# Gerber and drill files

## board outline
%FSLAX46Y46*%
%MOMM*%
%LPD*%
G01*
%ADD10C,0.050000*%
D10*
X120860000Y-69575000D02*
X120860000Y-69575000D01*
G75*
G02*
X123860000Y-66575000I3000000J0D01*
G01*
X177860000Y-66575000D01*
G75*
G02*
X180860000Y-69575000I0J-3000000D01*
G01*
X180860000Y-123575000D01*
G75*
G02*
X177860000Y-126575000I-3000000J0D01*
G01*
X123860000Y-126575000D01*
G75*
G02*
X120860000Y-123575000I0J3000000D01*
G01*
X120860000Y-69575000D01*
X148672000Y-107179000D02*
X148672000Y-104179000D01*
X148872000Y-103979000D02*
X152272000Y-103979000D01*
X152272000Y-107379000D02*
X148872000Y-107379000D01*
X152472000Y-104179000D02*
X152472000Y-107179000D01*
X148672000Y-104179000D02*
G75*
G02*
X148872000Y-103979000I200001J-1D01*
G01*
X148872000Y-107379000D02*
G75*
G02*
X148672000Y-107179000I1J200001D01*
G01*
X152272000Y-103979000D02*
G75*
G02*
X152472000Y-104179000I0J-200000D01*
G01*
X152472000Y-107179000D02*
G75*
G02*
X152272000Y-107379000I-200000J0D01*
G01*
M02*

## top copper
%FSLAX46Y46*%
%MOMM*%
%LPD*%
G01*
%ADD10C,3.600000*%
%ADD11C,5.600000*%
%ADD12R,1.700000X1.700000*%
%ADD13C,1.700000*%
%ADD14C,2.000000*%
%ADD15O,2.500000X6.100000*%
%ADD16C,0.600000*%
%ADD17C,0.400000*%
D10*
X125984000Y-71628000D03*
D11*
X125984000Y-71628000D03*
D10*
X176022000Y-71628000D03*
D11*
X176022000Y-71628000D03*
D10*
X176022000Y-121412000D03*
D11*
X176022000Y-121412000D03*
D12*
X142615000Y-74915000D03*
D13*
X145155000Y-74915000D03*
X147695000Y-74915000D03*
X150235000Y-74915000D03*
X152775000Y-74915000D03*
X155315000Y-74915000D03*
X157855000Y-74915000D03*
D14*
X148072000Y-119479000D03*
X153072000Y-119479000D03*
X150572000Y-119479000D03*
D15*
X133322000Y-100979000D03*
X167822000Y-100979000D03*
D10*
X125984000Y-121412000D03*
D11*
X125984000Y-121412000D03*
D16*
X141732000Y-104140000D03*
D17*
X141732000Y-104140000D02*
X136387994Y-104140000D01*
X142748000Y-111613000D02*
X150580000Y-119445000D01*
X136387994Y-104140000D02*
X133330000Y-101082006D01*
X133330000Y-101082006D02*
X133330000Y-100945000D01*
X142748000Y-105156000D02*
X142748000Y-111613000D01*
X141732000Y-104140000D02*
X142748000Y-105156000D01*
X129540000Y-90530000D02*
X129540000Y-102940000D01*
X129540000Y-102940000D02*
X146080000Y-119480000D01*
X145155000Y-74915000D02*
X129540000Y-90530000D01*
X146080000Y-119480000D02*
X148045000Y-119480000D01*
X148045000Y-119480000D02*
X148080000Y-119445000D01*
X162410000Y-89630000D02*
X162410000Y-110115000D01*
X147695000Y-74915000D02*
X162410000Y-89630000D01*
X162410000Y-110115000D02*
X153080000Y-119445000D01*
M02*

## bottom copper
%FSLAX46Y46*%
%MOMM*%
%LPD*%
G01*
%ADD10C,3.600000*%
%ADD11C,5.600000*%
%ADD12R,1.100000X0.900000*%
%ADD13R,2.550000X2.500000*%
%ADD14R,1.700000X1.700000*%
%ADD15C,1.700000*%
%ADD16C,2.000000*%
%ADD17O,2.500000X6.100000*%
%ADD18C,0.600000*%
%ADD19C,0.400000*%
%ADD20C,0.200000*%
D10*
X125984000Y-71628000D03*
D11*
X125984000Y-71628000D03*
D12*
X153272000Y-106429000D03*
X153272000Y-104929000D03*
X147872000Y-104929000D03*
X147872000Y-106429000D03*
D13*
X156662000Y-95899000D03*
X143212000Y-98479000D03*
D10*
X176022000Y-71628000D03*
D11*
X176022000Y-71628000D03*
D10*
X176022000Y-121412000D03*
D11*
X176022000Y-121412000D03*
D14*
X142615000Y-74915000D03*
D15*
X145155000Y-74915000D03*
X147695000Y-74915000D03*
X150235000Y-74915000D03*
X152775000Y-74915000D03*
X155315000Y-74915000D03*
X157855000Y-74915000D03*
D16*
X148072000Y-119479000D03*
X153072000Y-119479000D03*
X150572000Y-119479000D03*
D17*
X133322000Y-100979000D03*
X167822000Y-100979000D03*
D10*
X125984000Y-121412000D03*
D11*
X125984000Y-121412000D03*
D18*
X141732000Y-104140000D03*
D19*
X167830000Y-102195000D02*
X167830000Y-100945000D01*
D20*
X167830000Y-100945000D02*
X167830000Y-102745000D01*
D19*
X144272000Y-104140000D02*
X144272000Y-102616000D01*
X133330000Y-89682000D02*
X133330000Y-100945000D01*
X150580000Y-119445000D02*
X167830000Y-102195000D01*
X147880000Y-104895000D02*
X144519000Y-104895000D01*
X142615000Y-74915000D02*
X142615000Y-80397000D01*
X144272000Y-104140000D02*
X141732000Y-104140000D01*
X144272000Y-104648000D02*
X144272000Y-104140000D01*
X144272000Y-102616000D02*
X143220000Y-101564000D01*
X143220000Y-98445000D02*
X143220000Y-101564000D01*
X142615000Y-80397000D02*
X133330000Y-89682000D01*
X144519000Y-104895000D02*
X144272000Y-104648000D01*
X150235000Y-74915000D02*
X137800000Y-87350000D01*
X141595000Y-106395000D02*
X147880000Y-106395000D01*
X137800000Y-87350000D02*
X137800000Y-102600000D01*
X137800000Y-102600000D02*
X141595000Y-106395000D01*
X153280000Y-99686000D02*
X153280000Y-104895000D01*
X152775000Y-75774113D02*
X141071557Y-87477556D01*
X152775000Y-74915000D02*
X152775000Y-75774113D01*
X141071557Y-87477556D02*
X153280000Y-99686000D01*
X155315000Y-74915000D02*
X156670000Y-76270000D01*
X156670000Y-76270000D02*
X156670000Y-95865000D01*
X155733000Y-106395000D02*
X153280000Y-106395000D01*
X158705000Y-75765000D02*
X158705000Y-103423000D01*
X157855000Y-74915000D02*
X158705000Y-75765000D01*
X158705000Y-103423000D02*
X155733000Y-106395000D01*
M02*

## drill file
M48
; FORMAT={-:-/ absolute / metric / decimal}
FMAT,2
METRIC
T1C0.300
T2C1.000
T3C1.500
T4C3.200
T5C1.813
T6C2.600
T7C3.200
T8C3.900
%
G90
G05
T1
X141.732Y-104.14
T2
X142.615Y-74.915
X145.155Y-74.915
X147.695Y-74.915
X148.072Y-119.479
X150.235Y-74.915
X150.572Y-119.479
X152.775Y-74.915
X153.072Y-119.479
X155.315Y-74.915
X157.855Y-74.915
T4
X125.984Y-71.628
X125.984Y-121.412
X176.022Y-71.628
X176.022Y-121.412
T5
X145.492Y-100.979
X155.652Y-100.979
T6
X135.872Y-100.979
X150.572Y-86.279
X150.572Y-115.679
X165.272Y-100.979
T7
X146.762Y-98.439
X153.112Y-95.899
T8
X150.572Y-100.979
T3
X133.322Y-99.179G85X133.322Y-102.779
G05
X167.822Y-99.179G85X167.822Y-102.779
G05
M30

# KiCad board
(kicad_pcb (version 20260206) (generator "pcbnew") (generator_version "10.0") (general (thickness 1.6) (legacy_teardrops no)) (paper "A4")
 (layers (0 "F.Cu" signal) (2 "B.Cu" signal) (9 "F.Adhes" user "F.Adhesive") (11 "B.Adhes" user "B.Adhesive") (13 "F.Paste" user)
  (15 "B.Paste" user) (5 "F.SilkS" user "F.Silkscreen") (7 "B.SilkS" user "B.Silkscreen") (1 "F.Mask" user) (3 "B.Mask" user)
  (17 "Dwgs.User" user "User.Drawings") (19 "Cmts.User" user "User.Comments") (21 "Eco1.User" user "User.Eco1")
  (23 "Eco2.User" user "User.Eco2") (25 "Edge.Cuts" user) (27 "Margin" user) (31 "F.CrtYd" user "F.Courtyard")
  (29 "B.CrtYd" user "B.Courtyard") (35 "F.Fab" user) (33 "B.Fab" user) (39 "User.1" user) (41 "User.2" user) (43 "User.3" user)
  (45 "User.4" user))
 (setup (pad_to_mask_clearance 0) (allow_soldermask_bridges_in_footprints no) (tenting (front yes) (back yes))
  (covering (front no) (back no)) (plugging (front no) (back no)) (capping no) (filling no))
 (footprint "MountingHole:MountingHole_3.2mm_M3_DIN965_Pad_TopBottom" (layer "F.Cu") (at 125.984 71.628)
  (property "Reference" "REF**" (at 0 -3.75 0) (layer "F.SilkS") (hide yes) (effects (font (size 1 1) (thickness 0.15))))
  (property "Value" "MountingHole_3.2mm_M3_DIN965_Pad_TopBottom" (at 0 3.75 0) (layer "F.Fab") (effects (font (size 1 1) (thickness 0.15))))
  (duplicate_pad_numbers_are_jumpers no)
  (pad "1" thru_hole circle (at 0 0) (size 3.6 3.6) (drill 3.2) (layers "*.Cu" "*.Mask") (remove_unused_layers no) (zone_connect 2))
  (pad "1" connect circle (at 0 0) (size 5.6 5.6) (layers "F.Cu" "F.Mask") (zone_connect 2))
  (pad "1" connect circle (at 0 0) (size 5.6 5.6) (layers "B.Cu" "B.Mask") (zone_connect 2)))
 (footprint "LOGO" (layer "F.Cu") (at 170.18 84.074 -8)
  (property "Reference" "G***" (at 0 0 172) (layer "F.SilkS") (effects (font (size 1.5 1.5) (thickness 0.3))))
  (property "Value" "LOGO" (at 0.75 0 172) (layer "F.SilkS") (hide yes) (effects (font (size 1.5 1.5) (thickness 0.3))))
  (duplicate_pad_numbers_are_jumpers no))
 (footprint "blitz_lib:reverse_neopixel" (layer "F.Cu") (at 150.572 100.979)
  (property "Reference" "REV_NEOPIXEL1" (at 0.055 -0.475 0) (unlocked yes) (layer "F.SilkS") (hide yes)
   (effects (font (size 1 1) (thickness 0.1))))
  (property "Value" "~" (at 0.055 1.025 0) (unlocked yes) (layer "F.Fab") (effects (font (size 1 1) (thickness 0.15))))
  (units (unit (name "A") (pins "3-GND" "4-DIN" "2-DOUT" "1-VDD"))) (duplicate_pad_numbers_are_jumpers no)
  (fp_line (start -1.9 6.2) (end -1.9 3.2) (stroke (width 0.05) (type solid)) (layer "Edge.Cuts"))
  (fp_line (start -1.7 3) (end 1.7 3) (stroke (width 0.05) (type solid)) (layer "Edge.Cuts"))
  (fp_line (start 1.7 6.4) (end -1.7 6.4) (stroke (width 0.05) (type solid)) (layer "Edge.Cuts"))
  (fp_line (start 1.9 3.2) (end 1.9 6.2) (stroke (width 0.05) (type solid)) (layer "Edge.Cuts"))
  (fp_arc (start -1.9 3.2) (mid -1.841421 3.058579) (end -1.7 3) (stroke (width 0.05) (type solid)) (layer "Edge.Cuts"))
  (fp_arc (start -1.7 6.4) (mid -1.841421 6.341421) (end -1.9 6.2) (stroke (width 0.05) (type solid)) (layer "Edge.Cuts"))
  (fp_arc (start 1.7 3) (mid 1.841421 3.058579) (end 1.9 3.2) (stroke (width 0.05) (type solid)) (layer "Edge.Cuts"))
  (fp_arc (start 1.9 6.2) (mid 1.841421 6.341421) (end 1.7 6.4) (stroke (width 0.05) (type solid)) (layer "Edge.Cuts"))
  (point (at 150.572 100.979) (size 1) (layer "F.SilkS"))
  (pad "1-VDD" smd rect (at 2.7 5.45) (size 1.1 0.9) (layers "B.Cu" "B.Mask" "B.Paste") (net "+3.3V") (solder_mask_margin 0.1016)
   (solder_paste_margin 0) (thermal_bridge_angle 0)
   (padstack (mode front_inner_back)
    (layer "Inner" (shape rect) (size 1.1 0.9) (zone_connect -1)) (layer "B.Cu" (shape rect) (size 1.1 0.9) (zone_connect -1))))
  (pad "2-DOUT" smd rect (at 2.7 3.95) (size 1.1 0.9) (layers "B.Cu" "B.Mask" "B.Paste") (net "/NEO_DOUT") (solder_mask_margin 0.1016)
   (solder_paste_margin 0) (thermal_bridge_angle 0)
   (padstack (mode front_inner_back)
    (layer "Inner" (shape rect) (size 1.1 0.9) (zone_connect -1)) (layer "B.Cu" (shape rect) (size 1.1 0.9) (zone_connect -1))))
  (pad "3-GND" smd rect (at -2.7 3.95) (size 1.1 0.9) (layers "B.Cu" "B.Mask" "B.Paste") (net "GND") (solder_mask_margin 0.1016)
   (solder_paste_margin 0) (thermal_bridge_angle 0)
   (padstack (mode front_inner_back)
    (layer "Inner" (shape rect) (size 1.1 0.9) (zone_connect -1)) (layer "B.Cu" (shape rect) (size 1.1 0.9) (zone_connect -1))))
  (pad "4-DIN" smd rect (at -2.7 5.45) (size 1.1 0.9) (layers "B.Cu" "B.Mask" "B.Paste") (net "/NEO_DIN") (solder_mask_margin 0.1016)
   (solder_paste_margin 0) (thermal_bridge_angle 0)
   (padstack (mode front_inner_back)
    (layer "Inner" (shape rect) (size 1.1 0.9) (zone_connect -1)) (layer "B.Cu" (shape rect) (size 1.1 0.9) (zone_connect -1))))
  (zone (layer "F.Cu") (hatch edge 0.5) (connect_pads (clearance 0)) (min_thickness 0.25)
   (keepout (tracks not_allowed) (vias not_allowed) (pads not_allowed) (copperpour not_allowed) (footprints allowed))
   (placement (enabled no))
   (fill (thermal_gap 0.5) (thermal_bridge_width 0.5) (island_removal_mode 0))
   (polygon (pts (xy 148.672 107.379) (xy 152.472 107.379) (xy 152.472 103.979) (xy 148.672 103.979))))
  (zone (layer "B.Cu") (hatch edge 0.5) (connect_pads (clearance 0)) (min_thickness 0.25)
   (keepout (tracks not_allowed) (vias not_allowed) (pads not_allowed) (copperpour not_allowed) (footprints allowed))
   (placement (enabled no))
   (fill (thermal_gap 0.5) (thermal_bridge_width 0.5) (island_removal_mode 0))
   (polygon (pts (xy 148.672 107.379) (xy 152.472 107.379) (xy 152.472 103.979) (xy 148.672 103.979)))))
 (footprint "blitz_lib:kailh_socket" (layer "F.Cu") (at 150.572 100.979)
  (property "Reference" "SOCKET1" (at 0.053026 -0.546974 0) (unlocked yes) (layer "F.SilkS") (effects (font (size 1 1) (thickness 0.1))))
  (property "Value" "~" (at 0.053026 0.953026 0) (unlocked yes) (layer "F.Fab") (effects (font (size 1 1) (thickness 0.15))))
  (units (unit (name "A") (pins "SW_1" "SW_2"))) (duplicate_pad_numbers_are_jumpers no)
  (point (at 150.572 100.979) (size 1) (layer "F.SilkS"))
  (pad "" np_thru_hole circle (at -5.08 0) (size 1.8135 1.8135) (drill 1.8135) (layers "*.Cu" "*.Mask"))
  (pad "" np_thru_hole circle (at -3.81 -2.54) (size 3.2 3.2) (drill 3.2) (layers "*.Cu" "*.Mask"))
  (pad "" np_thru_hole circle (at 0 0) (size 3.9 3.9) (drill 3.9) (layers "*.Cu" "*.Mask"))
  (pad "" np_thru_hole circle (at 2.54 -5.08) (size 3.2 3.2) (drill 3.2) (layers "*.Cu" "*.Mask"))
  (pad "" np_thru_hole circle (at 5.08 0) (size 1.8135 1.8135) (drill 1.8135) (layers "*.Cu" "*.Mask"))
  (pad "SW_1" smd rect (at 6.09 -5.08 180) (size 2.55 2.5) (layers "B.Cu" "B.Mask" "B.Paste") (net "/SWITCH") (solder_mask_margin 0.1016)
   (solder_paste_margin 0) (thermal_bridge_angle 0))
  (pad "SW_2" smd rect (at -7.36 -2.5 180) (size 2.55 2.5) (layers "B.Cu" "B.Mask" "B.Paste") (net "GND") (solder_mask_margin 0.1016)
   (solder_paste_margin 0) (thermal_bridge_angle 0)))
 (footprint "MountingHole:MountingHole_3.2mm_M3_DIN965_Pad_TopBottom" (layer "F.Cu") (at 176.022 71.628)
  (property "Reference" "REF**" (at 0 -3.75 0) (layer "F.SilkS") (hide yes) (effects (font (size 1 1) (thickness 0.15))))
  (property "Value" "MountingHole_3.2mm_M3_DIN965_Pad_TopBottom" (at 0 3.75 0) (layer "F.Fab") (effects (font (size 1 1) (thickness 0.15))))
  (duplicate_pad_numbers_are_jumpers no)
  (pad "1" thru_hole circle (at 0 0) (size 3.6 3.6) (drill 3.2) (layers "*.Cu" "*.Mask") (remove_unused_layers no) (zone_connect 2))
  (pad "1" connect circle (at 0 0) (size 5.6 5.6) (layers "F.Cu" "F.Mask") (zone_connect 2))
  (pad "1" connect circle (at 0 0) (size 5.6 5.6) (layers "B.Cu" "B.Mask") (zone_connect 2)))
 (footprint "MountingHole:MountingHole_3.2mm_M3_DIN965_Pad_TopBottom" (layer "F.Cu") (at 176.022 121.412)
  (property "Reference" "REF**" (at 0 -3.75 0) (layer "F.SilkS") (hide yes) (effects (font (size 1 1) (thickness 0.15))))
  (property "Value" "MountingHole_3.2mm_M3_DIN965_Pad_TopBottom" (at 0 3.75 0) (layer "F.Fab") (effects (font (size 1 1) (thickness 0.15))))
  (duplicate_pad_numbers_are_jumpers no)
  (pad "1" thru_hole circle (at 0 0) (size 3.6 3.6) (drill 3.2) (layers "*.Cu" "*.Mask") (remove_unused_layers no) (zone_connect 2))
  (pad "1" connect circle (at 0 0) (size 5.6 5.6) (layers "F.Cu" "F.Mask") (zone_connect 2))
  (pad "1" connect circle (at 0 0) (size 5.6 5.6) (layers "B.Cu" "B.Mask") (zone_connect 2)))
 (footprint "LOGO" (layer "F.Cu") (at 132.588 115.062 -45)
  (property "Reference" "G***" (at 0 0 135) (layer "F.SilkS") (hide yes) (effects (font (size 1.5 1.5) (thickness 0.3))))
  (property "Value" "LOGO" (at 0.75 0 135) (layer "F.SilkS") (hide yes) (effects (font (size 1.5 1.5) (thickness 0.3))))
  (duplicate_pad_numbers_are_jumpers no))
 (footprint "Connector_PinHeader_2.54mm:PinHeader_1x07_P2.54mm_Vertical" (layer "F.Cu") (at 142.615 74.915 90)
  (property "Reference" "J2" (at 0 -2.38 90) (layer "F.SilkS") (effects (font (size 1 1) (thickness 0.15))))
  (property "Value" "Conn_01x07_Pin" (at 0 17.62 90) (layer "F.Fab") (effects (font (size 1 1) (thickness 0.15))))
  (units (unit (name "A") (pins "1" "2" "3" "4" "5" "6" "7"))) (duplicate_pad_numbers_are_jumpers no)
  (pad "1" thru_hole rect (at 0 0 90) (size 1.7 1.7) (drill 1) (layers "*.Cu" "*.Mask") (remove_unused_layers no) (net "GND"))
  (pad "2" thru_hole circle (at 0 2.54 90) (size 1.7 1.7) (drill 1) (layers "*.Cu" "*.Mask") (remove_unused_layers no) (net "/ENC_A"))
  (pad "3" thru_hole circle (at 0 5.08 90) (size 1.7 1.7) (drill 1) (layers "*.Cu" "*.Mask") (remove_unused_layers no) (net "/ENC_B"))
  (pad "4" thru_hole circle (at 0 7.62 90) (size 1.7 1.7) (drill 1) (layers "*.Cu" "*.Mask") (remove_unused_layers no) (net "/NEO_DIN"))
  (pad "5" thru_hole circle (at 0 10.16 90) (size 1.7 1.7) (drill 1) (layers "*.Cu" "*.Mask") (remove_unused_layers no) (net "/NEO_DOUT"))
  (pad "6" thru_hole circle (at 0 12.7 90) (size 1.7 1.7) (drill 1) (layers "*.Cu" "*.Mask") (remove_unused_layers no) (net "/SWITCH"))
  (pad "7" thru_hole circle (at 0 15.24 90) (size 1.7 1.7) (drill 1) (layers "*.Cu" "*.Mask") (remove_unused_layers no) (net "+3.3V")))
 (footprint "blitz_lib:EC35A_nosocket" (layer "F.Cu") (at 150.572 100.979)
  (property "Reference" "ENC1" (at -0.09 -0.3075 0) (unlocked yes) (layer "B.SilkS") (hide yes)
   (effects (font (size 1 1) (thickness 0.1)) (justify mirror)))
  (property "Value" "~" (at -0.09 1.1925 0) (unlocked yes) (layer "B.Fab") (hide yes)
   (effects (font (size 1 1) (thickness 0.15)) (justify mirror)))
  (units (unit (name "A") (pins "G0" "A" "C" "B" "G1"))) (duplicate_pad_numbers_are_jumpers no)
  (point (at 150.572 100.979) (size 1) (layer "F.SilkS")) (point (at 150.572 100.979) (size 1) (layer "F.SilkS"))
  (pad "" np_thru_hole circle (at -14.7 0) (size 2.54 2.54) (drill 2.6) (layers "*.Cu" "*.Mask"))
  (pad "" np_thru_hole circle (at 0 -14.7) (size 2.6 2.6) (drill 2.6) (layers "*.Cu" "*.Mask"))
  (pad "" np_thru_hole circle (at 0 14.7) (size 2.6 2.6) (drill 2.6) (layers "*.Cu" "*.Mask"))
  (pad "" np_thru_hole circle (at 14.7 0) (size 2.6 2.6) (drill 2.6) (layers "*.Cu" "*.Mask"))
  (pad "A" thru_hole circle (at -2.5 18.5) (size 2 2) (drill 1) (layers "*.Cu" "*.Mask") (remove_unused_layers no) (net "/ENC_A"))
  (pad "B" thru_hole circle (at 2.5 18.5) (size 2 2) (drill 1) (layers "*.Cu" "*.Mask") (remove_unused_layers no) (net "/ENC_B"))
  (pad "C" thru_hole circle (at 0 18.5) (size 2 2) (drill 1) (layers "*.Cu" "*.Mask") (remove_unused_layers no) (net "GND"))
  (pad "G0" thru_hole oval (at -17.25 0) (size 2.5 6.1) (drill oval 1.5 5.1) (layers "*.Cu" "*.Mask") (remove_unused_layers no) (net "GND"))
  (pad "G1" thru_hole oval (at 17.25 0) (size 2.5 6.1) (drill oval 1.5 5.1) (layers "*.Cu" "*.Mask") (remove_unused_layers no) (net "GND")))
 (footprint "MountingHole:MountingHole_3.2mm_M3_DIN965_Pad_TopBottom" (layer "F.Cu") (at 125.984 121.412)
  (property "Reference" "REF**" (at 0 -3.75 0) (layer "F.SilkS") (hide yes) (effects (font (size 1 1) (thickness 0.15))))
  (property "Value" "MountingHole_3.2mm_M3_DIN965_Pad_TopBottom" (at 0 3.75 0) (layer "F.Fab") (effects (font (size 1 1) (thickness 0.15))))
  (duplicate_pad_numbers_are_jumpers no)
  (pad "1" thru_hole circle (at 0 0) (size 3.6 3.6) (drill 3.2) (layers "*.Cu" "*.Mask") (remove_unused_layers no) (zone_connect 2))
  (pad "1" connect circle (at 0 0) (size 5.6 5.6) (layers "F.Cu" "F.Mask") (zone_connect 2))
  (pad "1" connect circle (at 0 0) (size 5.6 5.6) (layers "B.Cu" "B.Mask") (zone_connect 2)))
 (gr_rect (start 120.86 66.575) (end 180.86 126.575) (radius 3) (stroke (width 0.05) (type solid)) (fill no) (layer "Edge.Cuts"))
 (segment (start 141.732 104.14) (end 136.387994 104.14) (width 0.4) (layer "F.Cu") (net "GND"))
 (segment (start 142.748 111.613) (end 150.58 119.445) (width 0.4) (layer "F.Cu") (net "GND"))
 (segment (start 136.387994 104.14) (end 133.33 101.082006) (width 0.4) (layer "F.Cu") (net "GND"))
 (segment (start 133.33 101.082006) (end 133.33 100.945) (width 0.4) (layer "F.Cu") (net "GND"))
 (segment (start 142.748 105.156) (end 142.748 111.613) (width 0.4) (layer "F.Cu") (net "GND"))
 (segment (start 141.732 104.14) (end 142.748 105.156) (width 0.4) (layer "F.Cu") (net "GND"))
 (via (at 141.732 104.14) (size 0.6) (drill 0.3) (layers "F.Cu" "B.Cu") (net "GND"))
 (segment (start 167.83 102.195) (end 167.83 100.945) (width 0.4) (layer "B.Cu") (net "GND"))
 (segment (start 167.83 100.945) (end 167.83 102.745) (width 0.2) (layer "B.Cu") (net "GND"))
 (segment (start 144.272 104.14) (end 144.272 102.616) (width 0.4) (layer "B.Cu") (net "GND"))
 (segment (start 133.33 89.682) (end 133.33 100.945) (width 0.4) (layer "B.Cu") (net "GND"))
 (segment (start 150.58 119.445) (end 167.83 102.195) (width 0.4) (layer "B.Cu") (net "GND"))
 (segment (start 147.88 104.895) (end 144.519 104.895) (width 0.4) (layer "B.Cu") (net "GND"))
 (segment (start 142.615 74.915) (end 142.615 80.397) (width 0.4) (layer "B.Cu") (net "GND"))
 (segment (start 144.272 104.14) (end 141.732 104.14) (width 0.4) (layer "B.Cu") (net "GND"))
 (segment (start 144.272 104.648) (end 144.272 104.14) (width 0.4) (layer "B.Cu") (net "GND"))
 (segment (start 144.272 102.616) (end 143.22 101.564) (width 0.4) (layer "B.Cu") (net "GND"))
 (segment (start 143.22 98.445) (end 143.22 101.564) (width 0.4) (layer "B.Cu") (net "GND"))
 (segment (start 142.615 80.397) (end 133.33 89.682) (width 0.4) (layer "B.Cu") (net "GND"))
 (segment (start 144.519 104.895) (end 144.272 104.648) (width 0.4) (layer "B.Cu") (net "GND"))
 (segment (start 129.54 90.53) (end 129.54 102.94) (width 0.4) (layer "F.Cu") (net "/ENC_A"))
 (segment (start 129.54 102.94) (end 146.08 119.48) (width 0.4) (layer "F.Cu") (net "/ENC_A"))
 (segment (start 145.155 74.915) (end 129.54 90.53) (width 0.4) (layer "F.Cu") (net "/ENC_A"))
 (segment (start 146.08 119.48) (end 148.045 119.48) (width 0.4) (layer "F.Cu") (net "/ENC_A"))
 (segment (start 148.045 119.48) (end 148.08 119.445) (width 0.4) (layer "F.Cu") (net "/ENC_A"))
 (segment (start 162.41 89.63) (end 162.41 110.115) (width 0.4) (layer "F.Cu") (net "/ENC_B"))
 (segment (start 147.695 74.915) (end 162.41 89.63) (width 0.4) (layer "F.Cu") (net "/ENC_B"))
 (segment (start 162.41 110.115) (end 153.08 119.445) (width 0.4) (layer "F.Cu") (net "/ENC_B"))
 (segment (start 150.235 74.915) (end 137.8 87.35) (width 0.4) (layer "B.Cu") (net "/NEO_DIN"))
 (segment (start 141.595 106.395) (end 147.88 106.395) (width 0.4) (layer "B.Cu") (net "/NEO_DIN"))
 (segment (start 137.8 87.35) (end 137.8 102.6) (width 0.4) (layer "B.Cu") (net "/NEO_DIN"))
 (segment (start 137.8 102.6) (end 141.595 106.395) (width 0.4) (layer "B.Cu") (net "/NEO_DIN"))
 (segment (start 153.28 99.686) (end 153.28 104.895) (width 0.4) (layer "B.Cu") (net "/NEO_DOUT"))
 (segment (start 152.775 75.774113) (end 141.071557 87.477556) (width 0.4) (layer "B.Cu") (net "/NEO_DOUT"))
 (segment (start 152.775 74.915) (end 152.775 75.774113) (width 0.4) (layer "B.Cu") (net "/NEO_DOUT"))
 (segment (start 141.071557 87.477556) (end 153.28 99.686) (width 0.4) (layer "B.Cu") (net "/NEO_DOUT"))
 (segment (start 155.315 74.915) (end 156.67 76.27) (width 0.4) (layer "B.Cu") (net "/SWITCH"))
 (segment (start 156.67 76.27) (end 156.67 95.865) (width 0.4) (layer "B.Cu") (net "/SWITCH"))
 (segment (start 155.733 106.395) (end 153.28 106.395) (width 0.4) (layer "B.Cu") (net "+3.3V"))
 (segment (start 158.705 75.765) (end 158.705 103.423) (width 0.4) (layer "B.Cu") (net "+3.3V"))
 (segment (start 157.855 74.915) (end 158.705 75.765) (width 0.4) (layer "B.Cu") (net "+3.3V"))
 (segment (start 158.705 103.423) (end 155.733 106.395) (width 0.4) (layer "B.Cu") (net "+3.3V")))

